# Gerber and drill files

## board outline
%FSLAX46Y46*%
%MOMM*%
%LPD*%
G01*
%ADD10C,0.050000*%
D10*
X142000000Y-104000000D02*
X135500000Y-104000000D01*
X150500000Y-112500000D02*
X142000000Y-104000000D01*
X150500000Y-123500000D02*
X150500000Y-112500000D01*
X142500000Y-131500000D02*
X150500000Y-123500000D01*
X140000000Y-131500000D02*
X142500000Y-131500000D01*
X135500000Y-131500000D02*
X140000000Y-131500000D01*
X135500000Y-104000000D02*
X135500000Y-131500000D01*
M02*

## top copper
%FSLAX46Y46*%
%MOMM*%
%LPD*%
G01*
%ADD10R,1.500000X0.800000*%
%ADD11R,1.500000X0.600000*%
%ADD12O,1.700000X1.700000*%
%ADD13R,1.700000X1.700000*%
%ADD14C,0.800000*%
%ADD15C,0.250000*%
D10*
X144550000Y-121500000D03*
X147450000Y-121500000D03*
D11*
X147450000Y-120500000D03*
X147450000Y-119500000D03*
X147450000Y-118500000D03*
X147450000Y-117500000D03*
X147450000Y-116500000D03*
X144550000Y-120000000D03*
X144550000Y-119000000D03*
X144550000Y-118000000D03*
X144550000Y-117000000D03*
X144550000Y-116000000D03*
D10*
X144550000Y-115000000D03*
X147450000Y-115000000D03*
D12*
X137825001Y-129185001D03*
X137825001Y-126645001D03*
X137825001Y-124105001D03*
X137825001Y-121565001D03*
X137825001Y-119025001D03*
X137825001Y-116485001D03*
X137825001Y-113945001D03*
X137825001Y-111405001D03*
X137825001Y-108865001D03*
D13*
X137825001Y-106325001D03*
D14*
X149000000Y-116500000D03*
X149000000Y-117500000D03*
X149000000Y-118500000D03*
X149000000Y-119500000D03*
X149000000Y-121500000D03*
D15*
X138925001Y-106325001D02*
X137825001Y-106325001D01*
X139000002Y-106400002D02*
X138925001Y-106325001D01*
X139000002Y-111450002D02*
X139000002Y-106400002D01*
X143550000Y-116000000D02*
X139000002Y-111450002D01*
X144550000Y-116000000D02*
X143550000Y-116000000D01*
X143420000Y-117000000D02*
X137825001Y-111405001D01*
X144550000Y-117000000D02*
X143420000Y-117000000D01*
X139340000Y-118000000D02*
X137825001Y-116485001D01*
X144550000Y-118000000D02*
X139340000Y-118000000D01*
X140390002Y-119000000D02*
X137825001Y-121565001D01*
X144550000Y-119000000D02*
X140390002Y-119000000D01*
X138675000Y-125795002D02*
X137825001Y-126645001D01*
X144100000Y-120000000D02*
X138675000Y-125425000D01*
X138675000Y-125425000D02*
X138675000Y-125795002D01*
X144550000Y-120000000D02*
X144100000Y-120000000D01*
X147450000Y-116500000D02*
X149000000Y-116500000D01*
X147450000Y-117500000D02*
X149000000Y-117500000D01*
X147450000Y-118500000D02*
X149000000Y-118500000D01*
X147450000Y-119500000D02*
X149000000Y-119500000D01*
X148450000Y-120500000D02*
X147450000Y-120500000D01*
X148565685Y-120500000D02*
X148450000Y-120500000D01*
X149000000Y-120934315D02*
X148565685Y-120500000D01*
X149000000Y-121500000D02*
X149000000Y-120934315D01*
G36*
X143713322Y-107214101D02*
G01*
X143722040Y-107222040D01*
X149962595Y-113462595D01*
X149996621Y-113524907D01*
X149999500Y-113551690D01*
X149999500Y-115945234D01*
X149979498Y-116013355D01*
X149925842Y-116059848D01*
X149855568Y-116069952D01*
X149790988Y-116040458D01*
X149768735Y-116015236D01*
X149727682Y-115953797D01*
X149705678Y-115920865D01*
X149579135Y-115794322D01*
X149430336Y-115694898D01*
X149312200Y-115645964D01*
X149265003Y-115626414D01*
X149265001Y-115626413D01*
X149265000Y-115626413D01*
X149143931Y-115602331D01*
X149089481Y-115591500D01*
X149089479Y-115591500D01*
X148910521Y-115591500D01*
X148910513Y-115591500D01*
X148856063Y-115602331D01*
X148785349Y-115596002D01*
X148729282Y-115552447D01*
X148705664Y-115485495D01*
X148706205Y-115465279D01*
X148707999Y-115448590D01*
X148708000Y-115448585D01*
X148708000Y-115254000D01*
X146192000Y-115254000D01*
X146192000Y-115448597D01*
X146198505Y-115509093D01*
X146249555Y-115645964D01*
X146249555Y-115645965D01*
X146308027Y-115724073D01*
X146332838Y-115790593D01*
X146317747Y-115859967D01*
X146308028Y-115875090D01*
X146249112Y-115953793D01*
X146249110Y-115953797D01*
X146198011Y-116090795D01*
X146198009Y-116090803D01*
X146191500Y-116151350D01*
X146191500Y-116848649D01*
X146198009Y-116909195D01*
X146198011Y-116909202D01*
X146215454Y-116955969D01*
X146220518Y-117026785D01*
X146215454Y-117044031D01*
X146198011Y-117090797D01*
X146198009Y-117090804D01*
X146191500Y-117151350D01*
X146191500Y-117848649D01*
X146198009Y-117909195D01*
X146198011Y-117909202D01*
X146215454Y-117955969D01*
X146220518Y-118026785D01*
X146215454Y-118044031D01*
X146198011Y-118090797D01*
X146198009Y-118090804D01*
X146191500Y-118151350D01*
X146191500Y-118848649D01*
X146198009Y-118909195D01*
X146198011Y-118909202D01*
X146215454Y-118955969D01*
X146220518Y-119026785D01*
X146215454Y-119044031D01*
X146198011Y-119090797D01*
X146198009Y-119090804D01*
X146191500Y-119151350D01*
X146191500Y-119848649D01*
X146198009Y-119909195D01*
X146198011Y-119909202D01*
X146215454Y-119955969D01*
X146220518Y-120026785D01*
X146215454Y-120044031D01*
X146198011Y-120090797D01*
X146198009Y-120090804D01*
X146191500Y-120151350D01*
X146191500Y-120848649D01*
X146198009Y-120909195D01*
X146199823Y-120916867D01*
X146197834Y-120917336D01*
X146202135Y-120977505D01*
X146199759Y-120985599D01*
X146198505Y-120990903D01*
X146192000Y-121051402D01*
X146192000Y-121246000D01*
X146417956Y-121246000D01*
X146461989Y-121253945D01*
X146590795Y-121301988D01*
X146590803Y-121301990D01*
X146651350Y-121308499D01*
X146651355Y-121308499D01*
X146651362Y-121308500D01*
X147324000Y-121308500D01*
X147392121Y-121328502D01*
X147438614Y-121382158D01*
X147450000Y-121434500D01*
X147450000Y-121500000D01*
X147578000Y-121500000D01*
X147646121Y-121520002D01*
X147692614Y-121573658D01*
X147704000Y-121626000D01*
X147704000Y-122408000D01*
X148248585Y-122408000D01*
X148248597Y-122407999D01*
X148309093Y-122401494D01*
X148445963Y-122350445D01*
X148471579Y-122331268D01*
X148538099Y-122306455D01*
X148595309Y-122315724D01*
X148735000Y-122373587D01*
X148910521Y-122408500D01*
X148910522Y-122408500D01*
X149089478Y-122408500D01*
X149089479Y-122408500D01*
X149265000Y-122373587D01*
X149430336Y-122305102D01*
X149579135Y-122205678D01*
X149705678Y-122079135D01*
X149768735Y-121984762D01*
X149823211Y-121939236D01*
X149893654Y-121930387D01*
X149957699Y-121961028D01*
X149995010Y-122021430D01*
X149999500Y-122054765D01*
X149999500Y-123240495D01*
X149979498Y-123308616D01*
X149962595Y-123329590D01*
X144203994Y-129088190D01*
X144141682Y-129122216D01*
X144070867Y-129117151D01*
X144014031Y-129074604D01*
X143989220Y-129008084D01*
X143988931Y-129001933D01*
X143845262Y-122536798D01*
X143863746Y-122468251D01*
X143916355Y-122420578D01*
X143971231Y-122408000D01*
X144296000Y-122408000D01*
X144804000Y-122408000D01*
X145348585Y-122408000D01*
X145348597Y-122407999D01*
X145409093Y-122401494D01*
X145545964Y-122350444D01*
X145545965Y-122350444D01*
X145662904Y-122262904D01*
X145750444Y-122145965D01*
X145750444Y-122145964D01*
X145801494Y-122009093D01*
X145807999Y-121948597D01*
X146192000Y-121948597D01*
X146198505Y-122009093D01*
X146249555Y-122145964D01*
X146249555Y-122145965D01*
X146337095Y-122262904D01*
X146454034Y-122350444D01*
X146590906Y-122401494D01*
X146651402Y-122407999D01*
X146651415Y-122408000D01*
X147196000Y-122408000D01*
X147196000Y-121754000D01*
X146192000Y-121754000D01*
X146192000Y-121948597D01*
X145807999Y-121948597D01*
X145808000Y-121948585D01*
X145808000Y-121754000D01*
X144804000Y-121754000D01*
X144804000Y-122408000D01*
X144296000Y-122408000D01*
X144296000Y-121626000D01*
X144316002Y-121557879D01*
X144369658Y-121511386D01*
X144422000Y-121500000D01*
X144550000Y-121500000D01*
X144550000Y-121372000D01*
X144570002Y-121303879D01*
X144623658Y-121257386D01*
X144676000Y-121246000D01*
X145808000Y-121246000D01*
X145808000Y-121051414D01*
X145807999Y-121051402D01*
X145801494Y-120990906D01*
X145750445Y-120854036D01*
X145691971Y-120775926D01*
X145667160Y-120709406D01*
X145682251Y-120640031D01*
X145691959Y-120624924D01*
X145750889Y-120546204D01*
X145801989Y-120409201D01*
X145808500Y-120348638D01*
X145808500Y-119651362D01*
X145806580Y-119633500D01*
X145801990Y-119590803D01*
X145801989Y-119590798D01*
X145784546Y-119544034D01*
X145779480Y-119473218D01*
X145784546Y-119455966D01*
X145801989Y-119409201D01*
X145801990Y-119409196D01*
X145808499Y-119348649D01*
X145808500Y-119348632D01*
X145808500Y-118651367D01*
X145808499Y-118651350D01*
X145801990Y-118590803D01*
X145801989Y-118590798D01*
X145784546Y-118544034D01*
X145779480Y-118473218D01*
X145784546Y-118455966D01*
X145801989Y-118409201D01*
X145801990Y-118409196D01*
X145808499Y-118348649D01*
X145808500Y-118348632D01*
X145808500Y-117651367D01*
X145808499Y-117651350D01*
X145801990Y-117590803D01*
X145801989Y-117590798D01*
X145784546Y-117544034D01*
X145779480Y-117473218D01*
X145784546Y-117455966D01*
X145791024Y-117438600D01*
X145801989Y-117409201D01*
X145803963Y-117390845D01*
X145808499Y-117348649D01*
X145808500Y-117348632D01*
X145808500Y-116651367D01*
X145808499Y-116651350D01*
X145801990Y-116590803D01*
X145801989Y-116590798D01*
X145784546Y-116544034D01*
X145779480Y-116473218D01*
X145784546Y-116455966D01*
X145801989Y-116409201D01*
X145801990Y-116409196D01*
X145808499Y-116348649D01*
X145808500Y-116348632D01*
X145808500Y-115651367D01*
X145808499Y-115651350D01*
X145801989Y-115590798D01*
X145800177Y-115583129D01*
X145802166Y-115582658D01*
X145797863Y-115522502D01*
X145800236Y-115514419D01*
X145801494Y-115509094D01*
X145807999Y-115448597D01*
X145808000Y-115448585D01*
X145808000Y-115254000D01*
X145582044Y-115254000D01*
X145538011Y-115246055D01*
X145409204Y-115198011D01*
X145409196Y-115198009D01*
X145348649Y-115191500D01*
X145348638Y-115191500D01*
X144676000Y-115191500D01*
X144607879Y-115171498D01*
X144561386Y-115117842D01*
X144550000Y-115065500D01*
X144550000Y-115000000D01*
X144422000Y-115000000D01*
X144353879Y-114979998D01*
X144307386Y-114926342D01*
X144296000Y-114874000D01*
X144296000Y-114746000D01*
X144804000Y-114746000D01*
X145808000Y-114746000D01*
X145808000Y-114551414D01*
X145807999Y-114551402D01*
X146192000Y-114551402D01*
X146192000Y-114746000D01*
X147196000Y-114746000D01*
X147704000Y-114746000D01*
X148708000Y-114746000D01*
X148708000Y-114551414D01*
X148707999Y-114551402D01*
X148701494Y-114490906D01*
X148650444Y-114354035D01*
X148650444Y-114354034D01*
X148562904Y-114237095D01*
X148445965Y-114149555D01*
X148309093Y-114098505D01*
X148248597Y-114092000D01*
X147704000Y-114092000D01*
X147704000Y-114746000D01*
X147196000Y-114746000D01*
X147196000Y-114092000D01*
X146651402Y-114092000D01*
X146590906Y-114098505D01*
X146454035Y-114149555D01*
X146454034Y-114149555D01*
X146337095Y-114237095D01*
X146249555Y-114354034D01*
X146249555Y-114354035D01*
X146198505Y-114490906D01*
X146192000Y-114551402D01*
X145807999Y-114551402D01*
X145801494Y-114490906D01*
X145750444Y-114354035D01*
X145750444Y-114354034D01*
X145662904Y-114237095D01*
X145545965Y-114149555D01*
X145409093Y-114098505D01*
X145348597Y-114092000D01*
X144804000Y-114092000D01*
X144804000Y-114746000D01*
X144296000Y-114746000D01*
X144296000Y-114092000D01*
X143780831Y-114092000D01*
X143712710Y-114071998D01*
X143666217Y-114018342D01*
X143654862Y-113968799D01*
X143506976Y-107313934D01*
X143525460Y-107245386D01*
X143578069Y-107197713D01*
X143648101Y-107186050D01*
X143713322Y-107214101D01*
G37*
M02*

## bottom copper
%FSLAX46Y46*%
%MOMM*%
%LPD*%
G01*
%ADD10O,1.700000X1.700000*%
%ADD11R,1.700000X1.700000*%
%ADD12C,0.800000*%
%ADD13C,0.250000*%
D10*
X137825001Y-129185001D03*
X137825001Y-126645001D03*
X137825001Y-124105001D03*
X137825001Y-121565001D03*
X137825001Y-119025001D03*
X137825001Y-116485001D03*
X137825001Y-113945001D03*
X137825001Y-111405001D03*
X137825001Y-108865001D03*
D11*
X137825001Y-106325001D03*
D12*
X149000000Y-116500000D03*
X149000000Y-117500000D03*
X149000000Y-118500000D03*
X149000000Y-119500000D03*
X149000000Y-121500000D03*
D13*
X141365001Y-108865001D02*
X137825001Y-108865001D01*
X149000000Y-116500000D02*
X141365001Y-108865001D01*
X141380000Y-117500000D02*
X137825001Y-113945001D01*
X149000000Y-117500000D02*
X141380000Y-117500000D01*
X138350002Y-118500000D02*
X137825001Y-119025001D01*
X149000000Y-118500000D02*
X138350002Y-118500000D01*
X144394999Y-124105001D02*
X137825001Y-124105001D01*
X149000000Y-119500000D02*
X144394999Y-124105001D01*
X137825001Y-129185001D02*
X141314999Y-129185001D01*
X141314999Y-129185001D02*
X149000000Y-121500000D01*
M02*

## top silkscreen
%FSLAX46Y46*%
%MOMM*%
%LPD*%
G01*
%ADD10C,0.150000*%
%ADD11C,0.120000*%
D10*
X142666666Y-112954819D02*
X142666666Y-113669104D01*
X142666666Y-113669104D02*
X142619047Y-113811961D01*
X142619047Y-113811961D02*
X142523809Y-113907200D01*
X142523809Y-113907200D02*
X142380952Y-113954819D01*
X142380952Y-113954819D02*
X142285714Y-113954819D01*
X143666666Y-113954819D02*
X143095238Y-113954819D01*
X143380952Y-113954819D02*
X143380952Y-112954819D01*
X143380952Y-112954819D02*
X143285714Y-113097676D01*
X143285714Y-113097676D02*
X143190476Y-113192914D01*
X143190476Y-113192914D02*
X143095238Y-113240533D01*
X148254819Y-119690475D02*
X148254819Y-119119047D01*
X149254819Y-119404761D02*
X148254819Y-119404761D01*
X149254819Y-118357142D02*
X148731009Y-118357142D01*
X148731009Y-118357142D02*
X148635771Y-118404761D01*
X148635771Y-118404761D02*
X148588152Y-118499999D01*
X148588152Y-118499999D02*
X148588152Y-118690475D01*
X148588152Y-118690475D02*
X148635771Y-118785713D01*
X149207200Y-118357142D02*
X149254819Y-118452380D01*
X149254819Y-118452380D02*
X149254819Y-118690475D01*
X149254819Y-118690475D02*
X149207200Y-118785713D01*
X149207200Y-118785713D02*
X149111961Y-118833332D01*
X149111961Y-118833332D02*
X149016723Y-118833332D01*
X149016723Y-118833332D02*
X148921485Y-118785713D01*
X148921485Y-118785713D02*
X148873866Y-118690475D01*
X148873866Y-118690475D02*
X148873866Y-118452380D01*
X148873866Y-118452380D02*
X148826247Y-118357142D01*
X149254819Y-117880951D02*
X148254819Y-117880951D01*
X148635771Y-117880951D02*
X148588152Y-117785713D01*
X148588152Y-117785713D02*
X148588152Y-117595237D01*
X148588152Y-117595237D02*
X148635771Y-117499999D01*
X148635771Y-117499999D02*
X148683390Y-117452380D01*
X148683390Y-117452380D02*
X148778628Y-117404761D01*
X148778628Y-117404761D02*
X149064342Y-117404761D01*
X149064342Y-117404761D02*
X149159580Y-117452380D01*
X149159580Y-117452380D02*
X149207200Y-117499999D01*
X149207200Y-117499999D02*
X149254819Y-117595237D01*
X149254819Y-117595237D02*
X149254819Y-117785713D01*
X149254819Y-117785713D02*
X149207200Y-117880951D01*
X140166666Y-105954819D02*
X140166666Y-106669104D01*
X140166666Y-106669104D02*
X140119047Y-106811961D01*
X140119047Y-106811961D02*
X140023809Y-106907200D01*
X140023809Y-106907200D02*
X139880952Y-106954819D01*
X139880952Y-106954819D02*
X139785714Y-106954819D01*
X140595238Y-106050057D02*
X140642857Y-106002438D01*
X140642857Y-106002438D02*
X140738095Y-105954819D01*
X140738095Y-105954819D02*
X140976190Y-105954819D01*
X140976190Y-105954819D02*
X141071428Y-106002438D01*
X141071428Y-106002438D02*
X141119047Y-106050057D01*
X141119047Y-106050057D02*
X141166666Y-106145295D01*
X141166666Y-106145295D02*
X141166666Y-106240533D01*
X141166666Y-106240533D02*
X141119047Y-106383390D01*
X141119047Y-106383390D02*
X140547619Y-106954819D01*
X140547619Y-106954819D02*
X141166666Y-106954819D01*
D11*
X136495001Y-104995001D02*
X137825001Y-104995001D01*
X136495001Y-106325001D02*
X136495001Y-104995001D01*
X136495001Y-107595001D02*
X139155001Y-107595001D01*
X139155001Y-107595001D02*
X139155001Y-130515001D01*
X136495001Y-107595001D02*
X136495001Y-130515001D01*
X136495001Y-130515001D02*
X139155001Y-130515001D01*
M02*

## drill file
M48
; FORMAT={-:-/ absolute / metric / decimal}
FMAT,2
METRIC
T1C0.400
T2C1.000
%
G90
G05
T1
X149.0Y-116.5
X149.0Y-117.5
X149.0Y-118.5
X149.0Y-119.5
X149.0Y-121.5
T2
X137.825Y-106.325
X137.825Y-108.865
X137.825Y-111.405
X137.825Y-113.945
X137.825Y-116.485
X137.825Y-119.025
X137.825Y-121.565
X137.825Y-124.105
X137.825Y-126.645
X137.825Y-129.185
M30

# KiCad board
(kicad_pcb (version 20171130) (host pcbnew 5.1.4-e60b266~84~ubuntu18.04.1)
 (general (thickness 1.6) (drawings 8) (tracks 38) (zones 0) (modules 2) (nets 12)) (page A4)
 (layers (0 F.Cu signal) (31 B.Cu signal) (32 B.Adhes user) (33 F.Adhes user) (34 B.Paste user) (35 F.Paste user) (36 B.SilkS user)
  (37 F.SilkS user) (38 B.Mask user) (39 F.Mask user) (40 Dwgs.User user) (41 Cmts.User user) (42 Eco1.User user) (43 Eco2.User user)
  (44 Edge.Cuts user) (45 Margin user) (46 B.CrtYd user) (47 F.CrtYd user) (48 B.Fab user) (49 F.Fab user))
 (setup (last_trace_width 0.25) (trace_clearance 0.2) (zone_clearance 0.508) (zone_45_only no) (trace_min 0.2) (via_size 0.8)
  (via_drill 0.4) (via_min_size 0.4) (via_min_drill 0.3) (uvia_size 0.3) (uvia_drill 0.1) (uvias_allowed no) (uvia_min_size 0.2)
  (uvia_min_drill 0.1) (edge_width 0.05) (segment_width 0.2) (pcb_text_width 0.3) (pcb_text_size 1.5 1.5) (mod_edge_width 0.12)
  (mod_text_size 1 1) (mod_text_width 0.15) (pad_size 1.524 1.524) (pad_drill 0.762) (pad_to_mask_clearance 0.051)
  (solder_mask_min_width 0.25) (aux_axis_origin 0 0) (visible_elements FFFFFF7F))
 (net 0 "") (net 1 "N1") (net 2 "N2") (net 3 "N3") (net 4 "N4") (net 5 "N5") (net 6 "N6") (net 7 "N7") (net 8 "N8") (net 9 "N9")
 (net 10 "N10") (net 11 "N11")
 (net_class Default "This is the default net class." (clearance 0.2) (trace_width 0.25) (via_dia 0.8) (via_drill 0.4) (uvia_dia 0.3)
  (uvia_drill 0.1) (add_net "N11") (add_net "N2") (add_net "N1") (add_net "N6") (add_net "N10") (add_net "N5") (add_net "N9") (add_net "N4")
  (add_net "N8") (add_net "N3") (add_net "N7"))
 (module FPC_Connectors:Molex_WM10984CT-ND (layer F.Cu) (at 146 115 270)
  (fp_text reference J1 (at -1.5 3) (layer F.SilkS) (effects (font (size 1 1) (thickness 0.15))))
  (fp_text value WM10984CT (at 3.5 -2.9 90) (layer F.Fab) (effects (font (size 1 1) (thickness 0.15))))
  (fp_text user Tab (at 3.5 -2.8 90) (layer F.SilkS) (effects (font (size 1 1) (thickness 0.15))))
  (pad 11 smd rect (at 6.5 1.45 270) (size 0.8 1.5) (layers F.Cu F.Paste F.Mask) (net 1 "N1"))
  (pad 11 smd rect (at 6.5 -1.45 270) (size 0.8 1.5) (layers F.Cu F.Paste F.Mask) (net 1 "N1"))
  (pad 10 smd rect (at 5.5 -1.45 270) (size 0.6 1.5) (layers F.Cu F.Paste F.Mask) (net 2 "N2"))
  (pad 8 smd rect (at 4.5 -1.45 270) (size 0.6 1.5) (layers F.Cu F.Paste F.Mask) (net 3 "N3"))
  (pad 6 smd rect (at 3.5 -1.45 270) (size 0.6 1.5) (layers F.Cu F.Paste F.Mask) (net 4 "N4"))
  (pad 4 smd rect (at 2.5 -1.45 270) (size 0.6 1.5) (layers F.Cu F.Paste F.Mask) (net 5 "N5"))
  (pad 2 smd rect (at 1.5 -1.45 270) (size 0.6 1.5) (layers F.Cu F.Paste F.Mask) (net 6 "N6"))
  (pad 9 smd rect (at 5 1.45 270) (size 0.6 1.5) (layers F.Cu F.Paste F.Mask) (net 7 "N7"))
  (pad 7 smd rect (at 4 1.45 270) (size 0.6 1.5) (layers F.Cu F.Paste F.Mask) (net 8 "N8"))
  (pad 5 smd rect (at 3 1.45 270) (size 0.6 1.5) (layers F.Cu F.Paste F.Mask) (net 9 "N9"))
  (pad 3 smd rect (at 2 1.45 270) (size 0.6 1.5) (layers F.Cu F.Paste F.Mask) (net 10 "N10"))
  (pad 1 smd rect (at 1 1.45 270) (size 0.6 1.5) (layers F.Cu F.Paste F.Mask) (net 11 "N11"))
  (pad 11 smd rect (at 0 1.45 270) (size 0.8 1.5) (layers F.Cu F.Paste F.Mask) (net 1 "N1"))
  (pad 11 smd rect (at 0 -1.45 270) (size 0.8 1.5) (layers F.Cu F.Paste F.Mask) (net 1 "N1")))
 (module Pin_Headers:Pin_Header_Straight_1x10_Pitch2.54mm (layer F.Cu) (at 137.825001 106.325001)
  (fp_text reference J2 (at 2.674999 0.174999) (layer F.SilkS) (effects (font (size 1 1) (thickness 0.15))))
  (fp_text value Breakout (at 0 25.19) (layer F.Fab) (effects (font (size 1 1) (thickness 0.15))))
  (fp_line (start -1.33 -1.33) (end 0 -1.33) (layer F.SilkS) (width 0.12))
  (fp_line (start -1.33 0) (end -1.33 -1.33) (layer F.SilkS) (width 0.12))
  (fp_line (start -1.33 1.27) (end 1.33 1.27) (layer F.SilkS) (width 0.12))
  (fp_line (start 1.33 1.27) (end 1.33 24.19) (layer F.SilkS) (width 0.12))
  (fp_line (start -1.33 1.27) (end -1.33 24.19) (layer F.SilkS) (width 0.12))
  (fp_line (start -1.33 24.19) (end 1.33 24.19) (layer F.SilkS) (width 0.12))
  (pad 10 thru_hole oval (at 0 22.86) (size 1.7 1.7) (drill 1) (layers *.Cu *.Mask) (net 2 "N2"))
  (pad 9 thru_hole oval (at 0 20.32) (size 1.7 1.7) (drill 1) (layers *.Cu *.Mask) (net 7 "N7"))
  (pad 8 thru_hole oval (at 0 17.78) (size 1.7 1.7) (drill 1) (layers *.Cu *.Mask) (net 3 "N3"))
  (pad 7 thru_hole oval (at 0 15.24) (size 1.7 1.7) (drill 1) (layers *.Cu *.Mask) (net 8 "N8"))
  (pad 6 thru_hole oval (at 0 12.7) (size 1.7 1.7) (drill 1) (layers *.Cu *.Mask) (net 4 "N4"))
  (pad 5 thru_hole oval (at 0 10.16) (size 1.7 1.7) (drill 1) (layers *.Cu *.Mask) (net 9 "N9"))
  (pad 4 thru_hole oval (at 0 7.62) (size 1.7 1.7) (drill 1) (layers *.Cu *.Mask) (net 5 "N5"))
  (pad 3 thru_hole oval (at 0 5.08) (size 1.7 1.7) (drill 1) (layers *.Cu *.Mask) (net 10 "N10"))
  (pad 2 thru_hole oval (at 0 2.54) (size 1.7 1.7) (drill 1) (layers *.Cu *.Mask) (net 6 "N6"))
  (pad 1 thru_hole rect (at 0 0) (size 1.7 1.7) (drill 1) (layers *.Cu *.Mask) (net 11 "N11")))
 (gr_line (start 142 104) (end 135.5 104) (layer Edge.Cuts) (width 0.05))
 (gr_line (start 150.5 112.5) (end 142 104) (layer Edge.Cuts) (width 0.05))
 (gr_line (start 150.5 123.5) (end 150.5 112.5) (layer Edge.Cuts) (width 0.05))
 (gr_line (start 142.5 131.5) (end 150.5 123.5) (layer Edge.Cuts) (width 0.05))
 (gr_line (start 140 131.5) (end 142.5 131.5) (layer Edge.Cuts) (width 0.05))
 (gr_line (start 135.5 131.5) (end 140 131.5) (layer Edge.Cuts) (width 0.05))
 (gr_line (start 135.5 104) (end 135.5 131.5) (layer Edge.Cuts) (width 0.05))
 (segment (start 138.925001 106.325001) (end 137.825001 106.325001) (width 0.25) (layer F.Cu) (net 11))
 (segment (start 139.000002 106.400002) (end 138.925001 106.325001) (width 0.25) (layer F.Cu) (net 11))
 (segment (start 139.000002 111.450002) (end 139.000002 106.400002) (width 0.25) (layer F.Cu) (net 11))
 (segment (start 143.55 116) (end 139.000002 111.450002) (width 0.25) (layer F.Cu) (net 11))
 (segment (start 144.55 116) (end 143.55 116) (width 0.25) (layer F.Cu) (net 11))
 (segment (start 143.42 117) (end 137.825001 111.405001) (width 0.25) (layer F.Cu) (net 10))
 (segment (start 144.55 117) (end 143.42 117) (width 0.25) (layer F.Cu) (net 10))
 (segment (start 139.34 118) (end 137.825001 116.485001) (width 0.25) (layer F.Cu) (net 9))
 (segment (start 144.55 118) (end 139.34 118) (width 0.25) (layer F.Cu) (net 9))
 (segment (start 140.390002 119) (end 137.825001 121.565001) (width 0.25) (layer F.Cu) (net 8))
 (segment (start 144.55 119) (end 140.390002 119) (width 0.25) (layer F.Cu) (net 8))
 (segment (start 138.675 125.795002) (end 137.825001 126.645001) (width 0.25) (layer F.Cu) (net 7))
 (segment (start 144.1 120) (end 138.675 125.425) (width 0.25) (layer F.Cu) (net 7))
 (segment (start 138.675 125.425) (end 138.675 125.795002) (width 0.25) (layer F.Cu) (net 7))
 (segment (start 144.55 120) (end 144.1 120) (width 0.25) (layer F.Cu) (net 7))
 (via (at 149 116.5) (size 0.8) (drill 0.4) (layers F.Cu B.Cu) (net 6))
 (segment (start 147.45 116.5) (end 149 116.5) (width 0.25) (layer F.Cu) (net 6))
 (segment (start 141.365001 108.865001) (end 137.825001 108.865001) (width 0.25) (layer B.Cu) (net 6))
 (segment (start 149 116.5) (end 141.365001 108.865001) (width 0.25) (layer B.Cu) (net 6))
 (via (at 149 117.5) (size 0.8) (drill 0.4) (layers F.Cu B.Cu) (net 5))
 (segment (start 147.45 117.5) (end 149 117.5) (width 0.25) (layer F.Cu) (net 5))
 (segment (start 141.38 117.5) (end 137.825001 113.945001) (width 0.25) (layer B.Cu) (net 5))
 (segment (start 149 117.5) (end 141.38 117.5) (width 0.25) (layer B.Cu) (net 5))
 (via (at 149 118.5) (size 0.8) (drill 0.4) (layers F.Cu B.Cu) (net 4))
 (segment (start 147.45 118.5) (end 149 118.5) (width 0.25) (layer F.Cu) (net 4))
 (segment (start 138.350002 118.5) (end 137.825001 119.025001) (width 0.25) (layer B.Cu) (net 4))
 (segment (start 149 118.5) (end 138.350002 118.5) (width 0.25) (layer B.Cu) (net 4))
 (via (at 149 119.5) (size 0.8) (drill 0.4) (layers F.Cu B.Cu) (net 3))
 (segment (start 147.45 119.5) (end 149 119.5) (width 0.25) (layer F.Cu) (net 3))
 (segment (start 144.394999 124.105001) (end 137.825001 124.105001) (width 0.25) (layer B.Cu) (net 3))
 (segment (start 149 119.5) (end 144.394999 124.105001) (width 0.25) (layer B.Cu) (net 3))
 (via (at 149 121.5) (size 0.8) (drill 0.4) (layers F.Cu B.Cu) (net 2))
 (segment (start 137.825001 129.185001) (end 141.314999 129.185001) (width 0.25) (layer B.Cu) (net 2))
 (segment (start 141.314999 129.185001) (end 149 121.5) (width 0.25) (layer B.Cu) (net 2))
 (segment (start 148.45 120.5) (end 147.45 120.5) (width 0.25) (layer F.Cu) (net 2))
 (segment (start 148.565685 120.5) (end 148.45 120.5) (width 0.25) (layer F.Cu) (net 2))
 (segment (start 149 120.934315) (end 148.565685 120.5) (width 0.25) (layer F.Cu) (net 2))
 (segment (start 149 121.5) (end 149 120.934315) (width 0.25) (layer F.Cu) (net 2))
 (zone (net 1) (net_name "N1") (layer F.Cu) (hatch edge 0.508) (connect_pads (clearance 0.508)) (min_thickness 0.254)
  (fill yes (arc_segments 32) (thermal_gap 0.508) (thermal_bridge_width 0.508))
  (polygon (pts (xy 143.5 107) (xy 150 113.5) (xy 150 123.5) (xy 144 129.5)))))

